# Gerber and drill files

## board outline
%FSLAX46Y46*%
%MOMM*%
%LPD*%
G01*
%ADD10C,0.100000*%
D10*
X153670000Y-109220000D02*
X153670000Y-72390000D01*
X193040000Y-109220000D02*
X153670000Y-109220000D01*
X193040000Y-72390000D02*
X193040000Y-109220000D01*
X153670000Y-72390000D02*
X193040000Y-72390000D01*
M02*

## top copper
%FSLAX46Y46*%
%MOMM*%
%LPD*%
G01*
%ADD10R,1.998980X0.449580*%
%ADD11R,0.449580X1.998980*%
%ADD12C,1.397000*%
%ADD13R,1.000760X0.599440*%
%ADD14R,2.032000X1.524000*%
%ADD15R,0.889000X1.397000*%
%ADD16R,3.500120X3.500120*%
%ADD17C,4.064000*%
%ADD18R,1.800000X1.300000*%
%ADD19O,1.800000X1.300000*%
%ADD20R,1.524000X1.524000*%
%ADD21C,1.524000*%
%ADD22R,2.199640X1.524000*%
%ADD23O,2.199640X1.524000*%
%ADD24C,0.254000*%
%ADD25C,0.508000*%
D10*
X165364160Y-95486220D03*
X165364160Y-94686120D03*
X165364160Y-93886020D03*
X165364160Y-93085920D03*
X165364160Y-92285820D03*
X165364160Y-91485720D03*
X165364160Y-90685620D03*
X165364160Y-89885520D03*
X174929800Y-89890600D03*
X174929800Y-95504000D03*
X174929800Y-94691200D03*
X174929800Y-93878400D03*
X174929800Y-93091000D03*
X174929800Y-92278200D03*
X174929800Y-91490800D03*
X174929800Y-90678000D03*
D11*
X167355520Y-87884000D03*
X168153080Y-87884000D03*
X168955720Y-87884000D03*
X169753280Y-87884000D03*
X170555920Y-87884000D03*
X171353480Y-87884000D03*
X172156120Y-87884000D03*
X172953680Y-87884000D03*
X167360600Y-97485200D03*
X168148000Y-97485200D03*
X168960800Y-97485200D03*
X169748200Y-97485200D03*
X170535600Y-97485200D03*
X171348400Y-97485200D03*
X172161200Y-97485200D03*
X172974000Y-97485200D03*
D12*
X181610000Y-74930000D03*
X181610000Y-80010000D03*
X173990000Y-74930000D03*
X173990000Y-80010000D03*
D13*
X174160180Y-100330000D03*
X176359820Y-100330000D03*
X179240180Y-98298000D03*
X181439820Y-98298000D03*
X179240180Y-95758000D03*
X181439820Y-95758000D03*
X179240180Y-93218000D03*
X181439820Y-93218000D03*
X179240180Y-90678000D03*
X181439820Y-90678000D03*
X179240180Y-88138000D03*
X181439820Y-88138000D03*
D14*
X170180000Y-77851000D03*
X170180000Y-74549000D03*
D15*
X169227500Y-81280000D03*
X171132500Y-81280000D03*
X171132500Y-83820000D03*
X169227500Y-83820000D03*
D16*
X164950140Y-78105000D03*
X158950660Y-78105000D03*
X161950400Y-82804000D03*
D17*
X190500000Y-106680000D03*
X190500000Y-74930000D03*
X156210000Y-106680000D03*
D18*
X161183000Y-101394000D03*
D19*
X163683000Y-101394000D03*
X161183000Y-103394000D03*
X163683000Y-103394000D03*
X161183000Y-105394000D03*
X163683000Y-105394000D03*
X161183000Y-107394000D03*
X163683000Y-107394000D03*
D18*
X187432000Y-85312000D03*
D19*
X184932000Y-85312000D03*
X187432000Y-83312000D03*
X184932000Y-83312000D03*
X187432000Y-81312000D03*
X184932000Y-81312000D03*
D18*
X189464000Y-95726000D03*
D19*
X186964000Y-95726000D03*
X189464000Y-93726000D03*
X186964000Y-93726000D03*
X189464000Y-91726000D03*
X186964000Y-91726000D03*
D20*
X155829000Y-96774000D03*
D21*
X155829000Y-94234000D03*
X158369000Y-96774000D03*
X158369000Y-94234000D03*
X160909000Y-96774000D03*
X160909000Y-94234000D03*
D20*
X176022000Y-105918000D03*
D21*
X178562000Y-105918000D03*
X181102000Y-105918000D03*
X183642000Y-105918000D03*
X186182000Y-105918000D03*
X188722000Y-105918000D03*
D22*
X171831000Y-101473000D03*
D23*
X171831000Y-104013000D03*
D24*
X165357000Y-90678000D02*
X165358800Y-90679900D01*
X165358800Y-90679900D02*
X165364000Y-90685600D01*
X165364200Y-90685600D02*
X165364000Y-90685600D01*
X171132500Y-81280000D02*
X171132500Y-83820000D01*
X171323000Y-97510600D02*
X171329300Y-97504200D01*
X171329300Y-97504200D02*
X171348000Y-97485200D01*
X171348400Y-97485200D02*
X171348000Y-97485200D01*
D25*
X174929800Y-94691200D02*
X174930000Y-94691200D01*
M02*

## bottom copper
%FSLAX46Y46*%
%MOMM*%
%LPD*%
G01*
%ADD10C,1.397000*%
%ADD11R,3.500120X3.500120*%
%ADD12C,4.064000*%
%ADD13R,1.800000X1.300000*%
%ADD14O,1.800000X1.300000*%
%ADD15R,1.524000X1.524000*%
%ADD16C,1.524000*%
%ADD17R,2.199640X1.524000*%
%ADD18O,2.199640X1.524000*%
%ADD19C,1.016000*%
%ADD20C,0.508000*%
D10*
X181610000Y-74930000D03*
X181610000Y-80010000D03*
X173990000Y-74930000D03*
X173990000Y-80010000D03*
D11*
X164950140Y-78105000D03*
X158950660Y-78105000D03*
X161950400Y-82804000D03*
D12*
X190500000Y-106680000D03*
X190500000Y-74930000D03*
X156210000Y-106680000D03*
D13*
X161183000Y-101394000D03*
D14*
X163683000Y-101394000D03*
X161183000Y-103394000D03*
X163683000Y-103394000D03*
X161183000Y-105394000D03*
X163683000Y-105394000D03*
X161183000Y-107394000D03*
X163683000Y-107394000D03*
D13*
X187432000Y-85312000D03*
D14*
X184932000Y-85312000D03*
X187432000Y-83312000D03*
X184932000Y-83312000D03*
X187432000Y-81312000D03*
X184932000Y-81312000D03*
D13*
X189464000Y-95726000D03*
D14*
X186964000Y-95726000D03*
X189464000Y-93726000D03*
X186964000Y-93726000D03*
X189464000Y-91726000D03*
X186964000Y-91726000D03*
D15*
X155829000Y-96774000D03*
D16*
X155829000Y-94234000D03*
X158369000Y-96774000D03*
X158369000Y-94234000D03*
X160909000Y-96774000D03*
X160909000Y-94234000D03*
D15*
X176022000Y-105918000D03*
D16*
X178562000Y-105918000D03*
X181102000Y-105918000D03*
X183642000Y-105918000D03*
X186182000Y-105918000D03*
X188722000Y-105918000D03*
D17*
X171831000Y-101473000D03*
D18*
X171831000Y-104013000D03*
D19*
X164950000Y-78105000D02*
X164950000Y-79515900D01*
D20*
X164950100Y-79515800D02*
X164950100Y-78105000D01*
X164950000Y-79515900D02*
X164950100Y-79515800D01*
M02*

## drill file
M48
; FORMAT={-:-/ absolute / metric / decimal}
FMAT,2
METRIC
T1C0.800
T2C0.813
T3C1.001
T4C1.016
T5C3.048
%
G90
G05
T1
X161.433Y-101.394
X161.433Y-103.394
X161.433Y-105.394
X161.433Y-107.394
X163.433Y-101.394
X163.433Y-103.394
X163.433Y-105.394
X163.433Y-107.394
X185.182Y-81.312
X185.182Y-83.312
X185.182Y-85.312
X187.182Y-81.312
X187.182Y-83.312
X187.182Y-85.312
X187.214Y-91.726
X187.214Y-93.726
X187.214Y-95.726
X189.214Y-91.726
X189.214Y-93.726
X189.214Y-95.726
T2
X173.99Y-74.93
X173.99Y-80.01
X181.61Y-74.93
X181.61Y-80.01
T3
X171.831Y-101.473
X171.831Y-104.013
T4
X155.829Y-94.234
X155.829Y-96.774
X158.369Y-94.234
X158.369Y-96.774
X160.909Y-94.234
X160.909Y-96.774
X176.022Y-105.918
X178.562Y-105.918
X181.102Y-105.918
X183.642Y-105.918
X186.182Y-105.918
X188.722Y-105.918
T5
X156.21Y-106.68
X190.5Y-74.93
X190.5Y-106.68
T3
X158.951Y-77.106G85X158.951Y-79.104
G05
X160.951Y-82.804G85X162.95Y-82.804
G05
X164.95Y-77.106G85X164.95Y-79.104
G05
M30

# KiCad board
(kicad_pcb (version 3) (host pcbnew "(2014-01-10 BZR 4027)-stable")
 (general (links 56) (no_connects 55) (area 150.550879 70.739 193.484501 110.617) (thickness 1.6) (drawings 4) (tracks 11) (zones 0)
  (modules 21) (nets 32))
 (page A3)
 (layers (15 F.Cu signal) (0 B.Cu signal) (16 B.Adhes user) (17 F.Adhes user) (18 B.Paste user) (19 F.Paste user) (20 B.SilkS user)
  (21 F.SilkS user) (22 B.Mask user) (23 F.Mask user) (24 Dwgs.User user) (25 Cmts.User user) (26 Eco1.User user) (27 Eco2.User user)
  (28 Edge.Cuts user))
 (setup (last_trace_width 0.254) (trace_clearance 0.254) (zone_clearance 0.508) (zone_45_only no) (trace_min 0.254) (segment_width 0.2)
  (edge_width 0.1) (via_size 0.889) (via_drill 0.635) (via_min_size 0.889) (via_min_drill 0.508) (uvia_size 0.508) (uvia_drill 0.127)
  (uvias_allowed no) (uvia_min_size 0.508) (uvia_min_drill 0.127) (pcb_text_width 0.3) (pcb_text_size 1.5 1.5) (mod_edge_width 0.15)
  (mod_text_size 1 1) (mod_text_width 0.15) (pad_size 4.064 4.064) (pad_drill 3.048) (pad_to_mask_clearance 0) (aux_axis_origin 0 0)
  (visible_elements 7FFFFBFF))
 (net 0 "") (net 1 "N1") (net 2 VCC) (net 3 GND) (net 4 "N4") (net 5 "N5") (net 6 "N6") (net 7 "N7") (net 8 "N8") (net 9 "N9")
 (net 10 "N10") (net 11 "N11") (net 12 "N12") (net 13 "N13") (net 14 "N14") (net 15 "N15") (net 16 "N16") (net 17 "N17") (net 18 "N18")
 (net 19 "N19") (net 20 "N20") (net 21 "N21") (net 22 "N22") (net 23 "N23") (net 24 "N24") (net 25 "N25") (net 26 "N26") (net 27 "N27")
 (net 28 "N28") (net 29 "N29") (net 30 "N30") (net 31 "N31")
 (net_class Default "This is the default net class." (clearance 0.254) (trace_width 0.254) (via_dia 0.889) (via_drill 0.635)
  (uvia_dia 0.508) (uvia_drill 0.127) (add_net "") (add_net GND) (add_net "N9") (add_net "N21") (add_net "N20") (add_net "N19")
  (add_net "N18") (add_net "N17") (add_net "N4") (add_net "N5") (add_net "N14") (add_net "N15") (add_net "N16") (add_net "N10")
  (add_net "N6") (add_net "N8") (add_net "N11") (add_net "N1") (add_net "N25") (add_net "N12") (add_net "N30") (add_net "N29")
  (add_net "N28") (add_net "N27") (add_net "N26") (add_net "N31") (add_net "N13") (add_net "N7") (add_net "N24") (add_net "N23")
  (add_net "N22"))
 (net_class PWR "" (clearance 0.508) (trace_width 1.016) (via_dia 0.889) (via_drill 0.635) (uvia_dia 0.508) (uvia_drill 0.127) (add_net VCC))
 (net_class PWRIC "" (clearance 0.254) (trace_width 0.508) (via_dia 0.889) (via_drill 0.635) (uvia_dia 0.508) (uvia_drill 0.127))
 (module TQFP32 (layer F.Cu) (at 170.18 92.71)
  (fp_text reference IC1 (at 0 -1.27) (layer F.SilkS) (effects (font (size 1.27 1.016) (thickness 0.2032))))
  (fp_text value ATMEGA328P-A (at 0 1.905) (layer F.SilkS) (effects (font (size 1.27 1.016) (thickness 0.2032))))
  (pad 8 smd rect (at -4.81584 2.77622) (size 1.99898 0.44958) (layers F.Cu F.Paste F.Mask) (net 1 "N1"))
  (pad 7 smd rect (at -4.81584 1.97612) (size 1.99898 0.44958) (layers F.Cu F.Paste F.Mask))
  (pad 6 smd rect (at -4.81584 1.17602) (size 1.99898 0.44958) (layers F.Cu F.Paste F.Mask) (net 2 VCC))
  (pad 5 smd rect (at -4.81584 0.37592) (size 1.99898 0.44958) (layers F.Cu F.Paste F.Mask) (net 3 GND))
  (pad 4 smd rect (at -4.81584 -0.42418) (size 1.99898 0.44958) (layers F.Cu F.Paste F.Mask) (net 2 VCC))
  (pad 3 smd rect (at -4.81584 -1.22428) (size 1.99898 0.44958) (layers F.Cu F.Paste F.Mask) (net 3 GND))
  (pad 2 smd rect (at -4.81584 -2.02438) (size 1.99898 0.44958) (layers F.Cu F.Paste F.Mask) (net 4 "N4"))
  (pad 1 smd rect (at -4.81584 -2.82448) (size 1.99898 0.44958) (layers F.Cu F.Paste F.Mask) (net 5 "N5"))
  (pad 24 smd rect (at 4.7498 -2.8194) (size 1.99898 0.44958) (layers F.Cu F.Paste F.Mask) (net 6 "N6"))
  (pad 17 smd rect (at 4.7498 2.794) (size 1.99898 0.44958) (layers F.Cu F.Paste F.Mask) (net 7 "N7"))
  (pad 18 smd rect (at 4.7498 1.9812) (size 1.99898 0.44958) (layers F.Cu F.Paste F.Mask) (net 2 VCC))
  (pad 19 smd rect (at 4.7498 1.1684) (size 1.99898 0.44958) (layers F.Cu F.Paste F.Mask))
  (pad 20 smd rect (at 4.7498 0.381) (size 1.99898 0.44958) (layers F.Cu F.Paste F.Mask))
  (pad 21 smd rect (at 4.7498 -0.4318) (size 1.99898 0.44958) (layers F.Cu F.Paste F.Mask) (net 3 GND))
  (pad 22 smd rect (at 4.7498 -1.2192) (size 1.99898 0.44958) (layers F.Cu F.Paste F.Mask))
  (pad 23 smd rect (at 4.7498 -2.032) (size 1.99898 0.44958) (layers F.Cu F.Paste F.Mask) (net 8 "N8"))
  (pad 32 smd rect (at -2.82448 -4.826) (size 0.44958 1.99898) (layers F.Cu F.Paste F.Mask) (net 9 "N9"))
  (pad 31 smd rect (at -2.02692 -4.826) (size 0.44958 1.99898) (layers F.Cu F.Paste F.Mask) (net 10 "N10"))
  (pad 30 smd rect (at -1.22428 -4.826) (size 0.44958 1.99898) (layers F.Cu F.Paste F.Mask) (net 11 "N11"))
  (pad 29 smd rect (at -0.42672 -4.826) (size 0.44958 1.99898) (layers F.Cu F.Paste F.Mask) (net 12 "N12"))
  (pad 28 smd rect (at 0.37592 -4.826) (size 0.44958 1.99898) (layers F.Cu F.Paste F.Mask) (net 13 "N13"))
  (pad 27 smd rect (at 1.17348 -4.826) (size 0.44958 1.99898) (layers F.Cu F.Paste F.Mask) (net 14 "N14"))
  (pad 26 smd rect (at 1.97612 -4.826) (size 0.44958 1.99898) (layers F.Cu F.Paste F.Mask) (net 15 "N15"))
  (pad 25 smd rect (at 2.77368 -4.826) (size 0.44958 1.99898) (layers F.Cu F.Paste F.Mask) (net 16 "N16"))
  (pad 9 smd rect (at -2.8194 4.7752) (size 0.44958 1.99898) (layers F.Cu F.Paste F.Mask) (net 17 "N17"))
  (pad 10 smd rect (at -2.032 4.7752) (size 0.44958 1.99898) (layers F.Cu F.Paste F.Mask) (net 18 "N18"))
  (pad 11 smd rect (at -1.2192 4.7752) (size 0.44958 1.99898) (layers F.Cu F.Paste F.Mask) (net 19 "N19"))
  (pad 12 smd rect (at -0.4318 4.7752) (size 0.44958 1.99898) (layers F.Cu F.Paste F.Mask) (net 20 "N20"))
  (pad 13 smd rect (at 0.3556 4.7752) (size 0.44958 1.99898) (layers F.Cu F.Paste F.Mask) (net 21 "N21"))
  (pad 14 smd rect (at 1.1684 4.7752) (size 0.44958 1.99898) (layers F.Cu F.Paste F.Mask) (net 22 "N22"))
  (pad 15 smd rect (at 1.9812 4.7752) (size 0.44958 1.99898) (layers F.Cu F.Paste F.Mask) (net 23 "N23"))
  (pad 16 smd rect (at 2.794 4.7752) (size 0.44958 1.99898) (layers F.Cu F.Paste F.Mask) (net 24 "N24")))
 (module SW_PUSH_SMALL (layer F.Cu) (at 177.8 77.47)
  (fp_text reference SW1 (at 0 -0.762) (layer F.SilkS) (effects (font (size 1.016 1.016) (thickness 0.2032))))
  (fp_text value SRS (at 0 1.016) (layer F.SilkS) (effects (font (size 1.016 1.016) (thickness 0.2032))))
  (pad 1 thru_hole circle (at 3.81 -2.54) (size 1.397 1.397) (drill 0.8128) (layers *.Cu *.Mask F.SilkS) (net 1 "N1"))
  (pad 2 thru_hole circle (at 3.81 2.54) (size 1.397 1.397) (drill 0.8128) (layers *.Cu *.Mask F.SilkS) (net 3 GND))
  (pad 1 thru_hole circle (at -3.81 -2.54) (size 1.397 1.397) (drill 0.8128) (layers *.Cu *.Mask F.SilkS) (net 1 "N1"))
  (pad 2 thru_hole circle (at -3.81 2.54) (size 1.397 1.397) (drill 0.8128) (layers *.Cu *.Mask F.SilkS) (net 3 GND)))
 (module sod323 (layer F.Cu) (at 175.26 100.33 180)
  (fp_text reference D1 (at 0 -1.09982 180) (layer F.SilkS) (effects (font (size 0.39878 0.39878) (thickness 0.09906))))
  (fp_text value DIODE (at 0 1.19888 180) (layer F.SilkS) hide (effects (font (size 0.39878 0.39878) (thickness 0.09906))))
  (pad 2 smd rect (at 1.09982 0 180) (size 1.00076 0.59944) (layers F.Cu F.Paste F.Mask) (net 20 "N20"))
  (pad 1 smd rect (at -1.09982 0 180) (size 1.00076 0.59944) (layers F.Cu F.Paste F.Mask) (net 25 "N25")))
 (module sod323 (layer F.Cu) (at 180.34 98.298 180)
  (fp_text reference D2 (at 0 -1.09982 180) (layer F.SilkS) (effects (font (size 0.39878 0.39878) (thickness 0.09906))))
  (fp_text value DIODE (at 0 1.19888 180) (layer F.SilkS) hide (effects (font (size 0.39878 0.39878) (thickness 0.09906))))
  (pad 2 smd rect (at 1.09982 0 180) (size 1.00076 0.59944) (layers F.Cu F.Paste F.Mask) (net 21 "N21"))
  (pad 1 smd rect (at -1.09982 0 180) (size 1.00076 0.59944) (layers F.Cu F.Paste F.Mask) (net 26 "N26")))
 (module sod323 (layer F.Cu) (at 180.34 95.758 180)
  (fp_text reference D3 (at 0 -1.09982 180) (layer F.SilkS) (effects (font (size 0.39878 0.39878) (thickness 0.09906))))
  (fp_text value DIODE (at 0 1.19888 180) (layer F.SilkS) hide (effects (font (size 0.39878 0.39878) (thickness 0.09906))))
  (pad 2 smd rect (at 1.09982 0 180) (size 1.00076 0.59944) (layers F.Cu F.Paste F.Mask) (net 22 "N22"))
  (pad 1 smd rect (at -1.09982 0 180) (size 1.00076 0.59944) (layers F.Cu F.Paste F.Mask) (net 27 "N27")))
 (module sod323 (layer F.Cu) (at 180.34 93.218 180)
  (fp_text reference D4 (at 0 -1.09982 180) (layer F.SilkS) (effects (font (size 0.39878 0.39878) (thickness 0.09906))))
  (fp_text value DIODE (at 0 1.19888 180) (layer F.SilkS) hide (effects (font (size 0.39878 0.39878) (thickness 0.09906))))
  (pad 2 smd rect (at 1.09982 0 180) (size 1.00076 0.59944) (layers F.Cu F.Paste F.Mask) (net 23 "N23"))
  (pad 1 smd rect (at -1.09982 0 180) (size 1.00076 0.59944) (layers F.Cu F.Paste F.Mask) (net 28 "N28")))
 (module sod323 (layer F.Cu) (at 180.34 90.678 180)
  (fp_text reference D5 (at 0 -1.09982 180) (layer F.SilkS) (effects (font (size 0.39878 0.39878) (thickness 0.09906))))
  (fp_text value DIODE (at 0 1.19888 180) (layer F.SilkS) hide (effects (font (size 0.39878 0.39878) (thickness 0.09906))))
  (pad 2 smd rect (at 1.09982 0 180) (size 1.00076 0.59944) (layers F.Cu F.Paste F.Mask) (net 24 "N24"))
  (pad 1 smd rect (at -1.09982 0 180) (size 1.00076 0.59944) (layers F.Cu F.Paste F.Mask) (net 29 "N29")))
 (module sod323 (layer F.Cu) (at 180.34 88.138 180)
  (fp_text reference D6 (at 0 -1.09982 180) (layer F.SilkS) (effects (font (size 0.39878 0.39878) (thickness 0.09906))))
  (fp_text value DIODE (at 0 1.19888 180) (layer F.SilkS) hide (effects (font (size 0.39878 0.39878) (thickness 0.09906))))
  (pad 2 smd rect (at 1.09982 0 180) (size 1.00076 0.59944) (layers F.Cu F.Paste F.Mask) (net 7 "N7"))
  (pad 1 smd rect (at -1.09982 0 180) (size 1.00076 0.59944) (layers F.Cu F.Paste F.Mask) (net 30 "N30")))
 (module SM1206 (layer F.Cu) (at 170.18 76.2 90)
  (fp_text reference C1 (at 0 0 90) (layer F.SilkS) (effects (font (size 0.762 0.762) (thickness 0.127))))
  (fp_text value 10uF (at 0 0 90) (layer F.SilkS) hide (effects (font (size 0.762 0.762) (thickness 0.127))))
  (pad 1 smd rect (at -1.651 0 90) (size 1.524 2.032) (layers F.Cu F.Paste F.Mask) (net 2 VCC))
  (pad 2 smd rect (at 1.651 0 90) (size 1.524 2.032) (layers F.Cu F.Paste F.Mask) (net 3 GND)))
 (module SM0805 (layer F.Cu) (at 170.18 81.28)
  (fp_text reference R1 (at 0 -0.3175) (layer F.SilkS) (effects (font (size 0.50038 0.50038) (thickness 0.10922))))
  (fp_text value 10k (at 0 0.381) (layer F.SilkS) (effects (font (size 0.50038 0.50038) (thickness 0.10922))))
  (pad 1 smd rect (at -0.9525 0) (size 0.889 1.397) (layers F.Cu F.Paste F.Mask) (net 2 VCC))
  (pad 2 smd rect (at 0.9525 0) (size 0.889 1.397) (layers F.Cu F.Paste F.Mask) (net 12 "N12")))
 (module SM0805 (layer F.Cu) (at 170.18 83.82 180)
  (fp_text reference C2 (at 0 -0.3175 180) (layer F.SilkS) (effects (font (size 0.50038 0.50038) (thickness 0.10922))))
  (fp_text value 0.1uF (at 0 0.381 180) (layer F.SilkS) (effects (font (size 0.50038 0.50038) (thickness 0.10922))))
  (pad 1 smd rect (at -0.9525 0 180) (size 0.889 1.397) (layers F.Cu F.Paste F.Mask) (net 12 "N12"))
  (pad 2 smd rect (at 0.9525 0 180) (size 0.889 1.397) (layers F.Cu F.Paste F.Mask) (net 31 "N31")))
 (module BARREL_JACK (layer F.Cu) (at 158.75 78.105)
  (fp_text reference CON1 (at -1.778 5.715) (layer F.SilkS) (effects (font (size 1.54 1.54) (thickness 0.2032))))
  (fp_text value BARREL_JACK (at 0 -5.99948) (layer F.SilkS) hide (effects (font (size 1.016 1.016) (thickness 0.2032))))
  (pad 1 thru_hole rect (at 6.20014 0) (size 3.50012 3.50012) (drill oval 1.00076 2.99974) (layers *.Cu *.Mask F.SilkS) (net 2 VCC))
  (pad 2 thru_hole rect (at 0.20066 0) (size 3.50012 3.50012) (drill oval 1.00076 2.99974) (layers *.Cu *.Mask F.SilkS) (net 3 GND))
  (pad 3 thru_hole rect (at 3.2004 4.699) (size 3.50012 3.50012) (drill oval 2.99974 1.00076) (layers *.Cu *.Mask F.SilkS) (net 3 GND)))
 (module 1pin (layer F.Cu) (at 190.5 106.68)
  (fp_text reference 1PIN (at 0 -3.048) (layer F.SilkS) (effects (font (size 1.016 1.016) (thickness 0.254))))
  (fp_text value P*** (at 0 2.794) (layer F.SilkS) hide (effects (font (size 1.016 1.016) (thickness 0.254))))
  (pad 1 thru_hole circle (at 0 0) (size 4.064 4.064) (drill 3.048) (layers *.Cu *.Mask F.SilkS)))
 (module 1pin (layer F.Cu) (at 190.5 74.93)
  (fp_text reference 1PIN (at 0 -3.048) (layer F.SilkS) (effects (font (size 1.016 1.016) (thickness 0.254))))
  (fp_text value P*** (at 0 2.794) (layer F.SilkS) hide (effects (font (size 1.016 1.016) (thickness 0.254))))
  (pad 1 thru_hole circle (at 0 0) (size 4.064 4.064) (drill 3.048) (layers *.Cu *.Mask F.SilkS)))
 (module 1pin (layer F.Cu) (at 156.21 106.68)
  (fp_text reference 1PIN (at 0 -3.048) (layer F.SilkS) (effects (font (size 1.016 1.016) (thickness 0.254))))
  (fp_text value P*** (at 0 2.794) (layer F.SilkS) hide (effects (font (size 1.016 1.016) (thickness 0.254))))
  (pad 1 thru_hole circle (at 0 0) (size 4.064 4.064) (drill 3.048) (layers *.Cu *.Mask F.SilkS) (clearance 1)))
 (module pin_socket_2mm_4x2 (layer F.Cu) (at 162.433 104.394 270)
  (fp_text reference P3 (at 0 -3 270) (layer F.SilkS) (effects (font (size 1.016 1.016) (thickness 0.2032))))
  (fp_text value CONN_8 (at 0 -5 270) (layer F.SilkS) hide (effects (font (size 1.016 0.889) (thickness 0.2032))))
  (pad 1 thru_hole rect (at -3 1 270) (size 1.3 1.8) (drill 0.8 (offset 0 0.25)) (layers *.Cu *.Mask F.SilkS) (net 11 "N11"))
  (pad 2 thru_hole oval (at -3 -1 270) (size 1.3 1.8) (drill 0.8 (offset 0 -0.25)) (layers *.Cu *.Mask F.SilkS) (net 10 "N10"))
  (pad 3 thru_hole oval (at -1 1 270) (size 1.3 1.8) (drill 0.8 (offset 0 0.25)) (layers *.Cu *.Mask F.SilkS) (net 9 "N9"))
  (pad 4 thru_hole oval (at -1 -1 270) (size 1.3 1.8) (drill 0.8 (offset 0 -0.25)) (layers *.Cu *.Mask F.SilkS) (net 5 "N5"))
  (pad 5 thru_hole oval (at 1 1 270) (size 1.3 1.8) (drill 0.8 (offset 0 0.25)) (layers *.Cu *.Mask F.SilkS) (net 4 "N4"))
  (pad 6 thru_hole oval (at 1 -1 270) (size 1.3 1.8) (drill 0.8 (offset 0 -0.25)) (layers *.Cu *.Mask F.SilkS) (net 17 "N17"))
  (pad 7 thru_hole oval (at 3 1 270) (size 1.3 1.8) (drill 0.8 (offset 0 0.25)) (layers *.Cu *.Mask F.SilkS) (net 18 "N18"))
  (pad 8 thru_hole oval (at 3 -1 270) (size 1.3 1.8) (drill 0.8 (offset 0 -0.25)) (layers *.Cu *.Mask F.SilkS) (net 19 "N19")))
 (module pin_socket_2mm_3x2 (layer F.Cu) (at 186.182 83.312 90)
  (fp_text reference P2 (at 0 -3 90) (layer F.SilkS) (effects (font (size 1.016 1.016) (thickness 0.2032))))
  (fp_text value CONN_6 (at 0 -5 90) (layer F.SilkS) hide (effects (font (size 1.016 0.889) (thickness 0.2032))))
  (pad 1 thru_hole rect (at -2 1 90) (size 1.3 1.8) (drill 0.8 (offset 0 0.25)) (layers *.Cu *.Mask F.SilkS) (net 8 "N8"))
  (pad 2 thru_hole oval (at -2 -1 90) (size 1.3 1.8) (drill 0.8 (offset 0 -0.25)) (layers *.Cu *.Mask F.SilkS) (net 6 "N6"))
  (pad 3 thru_hole oval (at 0 1 90) (size 1.3 1.8) (drill 0.8 (offset 0 0.25)) (layers *.Cu *.Mask F.SilkS) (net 16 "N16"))
  (pad 4 thru_hole oval (at 0 -1 90) (size 1.3 1.8) (drill 0.8 (offset 0 -0.25)) (layers *.Cu *.Mask F.SilkS) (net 15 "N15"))
  (pad 5 thru_hole oval (at 2 1 90) (size 1.3 1.8) (drill 0.8 (offset 0 0.25)) (layers *.Cu *.Mask F.SilkS) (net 14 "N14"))
  (pad 6 thru_hole oval (at 2 -1 90) (size 1.3 1.8) (drill 0.8 (offset 0 -0.25)) (layers *.Cu *.Mask F.SilkS) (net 13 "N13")))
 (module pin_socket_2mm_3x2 (layer F.Cu) (at 188.214 93.726 90)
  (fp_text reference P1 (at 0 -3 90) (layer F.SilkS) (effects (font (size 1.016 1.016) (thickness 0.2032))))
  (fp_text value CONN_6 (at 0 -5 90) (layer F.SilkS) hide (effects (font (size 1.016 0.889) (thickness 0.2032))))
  (pad 1 thru_hole rect (at -2 1 90) (size 1.3 1.8) (drill 0.8 (offset 0 0.25)) (layers *.Cu *.Mask F.SilkS) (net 25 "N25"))
  (pad 2 thru_hole oval (at -2 -1 90) (size 1.3 1.8) (drill 0.8 (offset 0 -0.25)) (layers *.Cu *.Mask F.SilkS) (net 26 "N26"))
  (pad 3 thru_hole oval (at 0 1 90) (size 1.3 1.8) (drill 0.8 (offset 0 0.25)) (layers *.Cu *.Mask F.SilkS) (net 27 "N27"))
  (pad 4 thru_hole oval (at 0 -1 90) (size 1.3 1.8) (drill 0.8 (offset 0 -0.25)) (layers *.Cu *.Mask F.SilkS) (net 28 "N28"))
  (pad 5 thru_hole oval (at 2 1 90) (size 1.3 1.8) (drill 0.8 (offset 0 0.25)) (layers *.Cu *.Mask F.SilkS) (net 29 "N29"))
  (pad 6 thru_hole oval (at 2 -1 90) (size 1.3 1.8) (drill 0.8 (offset 0 -0.25)) (layers *.Cu *.Mask F.SilkS) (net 30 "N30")))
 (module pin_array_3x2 (layer F.Cu) (at 158.369 95.504)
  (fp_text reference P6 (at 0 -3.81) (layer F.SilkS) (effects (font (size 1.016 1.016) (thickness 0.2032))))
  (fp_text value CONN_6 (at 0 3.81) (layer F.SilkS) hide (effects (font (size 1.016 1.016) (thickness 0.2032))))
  (pad 1 thru_hole rect (at -2.54 1.27) (size 1.524 1.524) (drill 1.016) (layers *.Cu *.Mask F.SilkS) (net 24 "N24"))
  (pad 2 thru_hole circle (at -2.54 -1.27) (size 1.524 1.524) (drill 1.016) (layers *.Cu *.Mask F.SilkS) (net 2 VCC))
  (pad 3 thru_hole circle (at 0 1.27) (size 1.524 1.524) (drill 1.016) (layers *.Cu *.Mask F.SilkS) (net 7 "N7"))
  (pad 4 thru_hole circle (at 0 -1.27) (size 1.524 1.524) (drill 1.016) (layers *.Cu *.Mask F.SilkS) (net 23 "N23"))
  (pad 5 thru_hole circle (at 2.54 1.27) (size 1.524 1.524) (drill 1.016) (layers *.Cu *.Mask F.SilkS) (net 12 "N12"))
  (pad 6 thru_hole circle (at 2.54 -1.27) (size 1.524 1.524) (drill 1.016) (layers *.Cu *.Mask F.SilkS) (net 3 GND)))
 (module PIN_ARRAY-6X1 (layer F.Cu) (at 182.372 105.918)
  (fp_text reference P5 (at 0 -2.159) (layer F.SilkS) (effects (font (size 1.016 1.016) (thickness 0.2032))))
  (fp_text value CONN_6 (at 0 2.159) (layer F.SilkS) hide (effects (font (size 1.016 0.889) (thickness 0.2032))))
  (pad 1 thru_hole rect (at -6.35 0) (size 1.524 1.524) (drill 1.016) (layers *.Cu *.Mask F.SilkS) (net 31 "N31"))
  (pad 2 thru_hole circle (at -3.81 0) (size 1.524 1.524) (drill 1.016) (layers *.Cu *.Mask F.SilkS) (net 10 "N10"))
  (pad 3 thru_hole circle (at -1.27 0) (size 1.524 1.524) (drill 1.016) (layers *.Cu *.Mask F.SilkS) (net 11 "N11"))
  (pad 4 thru_hole circle (at 1.27 0) (size 1.524 1.524) (drill 1.016) (layers *.Cu *.Mask F.SilkS) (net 2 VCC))
  (pad 5 thru_hole circle (at 3.81 0) (size 1.524 1.524) (drill 1.016) (layers *.Cu *.Mask F.SilkS) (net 3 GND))
  (pad 6 thru_hole circle (at 6.35 0) (size 1.524 1.524) (drill 1.016) (layers *.Cu *.Mask F.SilkS) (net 3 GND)))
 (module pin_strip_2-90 (layer F.Cu) (at 171.831 102.743 270)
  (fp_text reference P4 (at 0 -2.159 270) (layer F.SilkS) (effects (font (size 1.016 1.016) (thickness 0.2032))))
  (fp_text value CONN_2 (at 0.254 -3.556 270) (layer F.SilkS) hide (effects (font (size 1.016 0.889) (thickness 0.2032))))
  (pad 1 thru_hole rect (at -1.27 0 270) (size 1.524 2.19964) (drill 1.00076) (layers *.Cu *.Mask F.SilkS) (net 2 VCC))
  (pad 2 thru_hole oval (at 1.27 0 270) (size 1.524 2.19964) (drill 1.00076) (layers *.Cu *.Mask F.SilkS) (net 3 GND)))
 (gr_line (start 153.67 109.22) (end 153.67 72.39) (angle 90) (layer Edge.Cuts) (width 0.1))
 (gr_line (start 193.04 109.22) (end 153.67 109.22) (angle 90) (layer Edge.Cuts) (width 0.1))
 (gr_line (start 193.04 72.39) (end 193.04 109.22) (angle 90) (layer Edge.Cuts) (width 0.1))
 (gr_line (start 153.67 72.39) (end 193.04 72.39) (angle 90) (layer Edge.Cuts) (width 0.1))
 (segment (start 165.357 90.678) (end 165.3588 90.6799) (width 0.254) (layer F.Cu) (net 4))
 (segment (start 165.3588 90.6799) (end 165.364 90.6856) (width 0.254) (layer F.Cu) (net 4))
 (segment (start 165.3642 90.6856) (end 165.364 90.6856) (width 0.254) (layer F.Cu) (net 4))
 (segment (start 171.1325 81.28) (end 171.1325 83.82) (width 0.254) (layer F.Cu) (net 12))
 (segment (start 171.323 97.5106) (end 171.3293 97.5042) (width 0.254) (layer F.Cu) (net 22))
 (segment (start 171.3293 97.5042) (end 171.348 97.4852) (width 0.254) (layer F.Cu) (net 22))
 (segment (start 171.3484 97.4852) (end 171.348 97.4852) (width 0.254) (layer F.Cu) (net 22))
 (segment (start 174.9298 94.6912) (end 174.93 94.6912) (width 0.508) (layer F.Cu) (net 2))
 (segment (start 164.95 78.105) (end 164.95 79.5159) (width 1.016) (layer B.Cu) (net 2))
 (segment (start 164.9501 79.5158) (end 164.9501 78.105) (width 0.508) (layer B.Cu) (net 2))
 (segment (start 164.95 79.5159) (end 164.9501 79.5158) (width 0.508) (layer B.Cu) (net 2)))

